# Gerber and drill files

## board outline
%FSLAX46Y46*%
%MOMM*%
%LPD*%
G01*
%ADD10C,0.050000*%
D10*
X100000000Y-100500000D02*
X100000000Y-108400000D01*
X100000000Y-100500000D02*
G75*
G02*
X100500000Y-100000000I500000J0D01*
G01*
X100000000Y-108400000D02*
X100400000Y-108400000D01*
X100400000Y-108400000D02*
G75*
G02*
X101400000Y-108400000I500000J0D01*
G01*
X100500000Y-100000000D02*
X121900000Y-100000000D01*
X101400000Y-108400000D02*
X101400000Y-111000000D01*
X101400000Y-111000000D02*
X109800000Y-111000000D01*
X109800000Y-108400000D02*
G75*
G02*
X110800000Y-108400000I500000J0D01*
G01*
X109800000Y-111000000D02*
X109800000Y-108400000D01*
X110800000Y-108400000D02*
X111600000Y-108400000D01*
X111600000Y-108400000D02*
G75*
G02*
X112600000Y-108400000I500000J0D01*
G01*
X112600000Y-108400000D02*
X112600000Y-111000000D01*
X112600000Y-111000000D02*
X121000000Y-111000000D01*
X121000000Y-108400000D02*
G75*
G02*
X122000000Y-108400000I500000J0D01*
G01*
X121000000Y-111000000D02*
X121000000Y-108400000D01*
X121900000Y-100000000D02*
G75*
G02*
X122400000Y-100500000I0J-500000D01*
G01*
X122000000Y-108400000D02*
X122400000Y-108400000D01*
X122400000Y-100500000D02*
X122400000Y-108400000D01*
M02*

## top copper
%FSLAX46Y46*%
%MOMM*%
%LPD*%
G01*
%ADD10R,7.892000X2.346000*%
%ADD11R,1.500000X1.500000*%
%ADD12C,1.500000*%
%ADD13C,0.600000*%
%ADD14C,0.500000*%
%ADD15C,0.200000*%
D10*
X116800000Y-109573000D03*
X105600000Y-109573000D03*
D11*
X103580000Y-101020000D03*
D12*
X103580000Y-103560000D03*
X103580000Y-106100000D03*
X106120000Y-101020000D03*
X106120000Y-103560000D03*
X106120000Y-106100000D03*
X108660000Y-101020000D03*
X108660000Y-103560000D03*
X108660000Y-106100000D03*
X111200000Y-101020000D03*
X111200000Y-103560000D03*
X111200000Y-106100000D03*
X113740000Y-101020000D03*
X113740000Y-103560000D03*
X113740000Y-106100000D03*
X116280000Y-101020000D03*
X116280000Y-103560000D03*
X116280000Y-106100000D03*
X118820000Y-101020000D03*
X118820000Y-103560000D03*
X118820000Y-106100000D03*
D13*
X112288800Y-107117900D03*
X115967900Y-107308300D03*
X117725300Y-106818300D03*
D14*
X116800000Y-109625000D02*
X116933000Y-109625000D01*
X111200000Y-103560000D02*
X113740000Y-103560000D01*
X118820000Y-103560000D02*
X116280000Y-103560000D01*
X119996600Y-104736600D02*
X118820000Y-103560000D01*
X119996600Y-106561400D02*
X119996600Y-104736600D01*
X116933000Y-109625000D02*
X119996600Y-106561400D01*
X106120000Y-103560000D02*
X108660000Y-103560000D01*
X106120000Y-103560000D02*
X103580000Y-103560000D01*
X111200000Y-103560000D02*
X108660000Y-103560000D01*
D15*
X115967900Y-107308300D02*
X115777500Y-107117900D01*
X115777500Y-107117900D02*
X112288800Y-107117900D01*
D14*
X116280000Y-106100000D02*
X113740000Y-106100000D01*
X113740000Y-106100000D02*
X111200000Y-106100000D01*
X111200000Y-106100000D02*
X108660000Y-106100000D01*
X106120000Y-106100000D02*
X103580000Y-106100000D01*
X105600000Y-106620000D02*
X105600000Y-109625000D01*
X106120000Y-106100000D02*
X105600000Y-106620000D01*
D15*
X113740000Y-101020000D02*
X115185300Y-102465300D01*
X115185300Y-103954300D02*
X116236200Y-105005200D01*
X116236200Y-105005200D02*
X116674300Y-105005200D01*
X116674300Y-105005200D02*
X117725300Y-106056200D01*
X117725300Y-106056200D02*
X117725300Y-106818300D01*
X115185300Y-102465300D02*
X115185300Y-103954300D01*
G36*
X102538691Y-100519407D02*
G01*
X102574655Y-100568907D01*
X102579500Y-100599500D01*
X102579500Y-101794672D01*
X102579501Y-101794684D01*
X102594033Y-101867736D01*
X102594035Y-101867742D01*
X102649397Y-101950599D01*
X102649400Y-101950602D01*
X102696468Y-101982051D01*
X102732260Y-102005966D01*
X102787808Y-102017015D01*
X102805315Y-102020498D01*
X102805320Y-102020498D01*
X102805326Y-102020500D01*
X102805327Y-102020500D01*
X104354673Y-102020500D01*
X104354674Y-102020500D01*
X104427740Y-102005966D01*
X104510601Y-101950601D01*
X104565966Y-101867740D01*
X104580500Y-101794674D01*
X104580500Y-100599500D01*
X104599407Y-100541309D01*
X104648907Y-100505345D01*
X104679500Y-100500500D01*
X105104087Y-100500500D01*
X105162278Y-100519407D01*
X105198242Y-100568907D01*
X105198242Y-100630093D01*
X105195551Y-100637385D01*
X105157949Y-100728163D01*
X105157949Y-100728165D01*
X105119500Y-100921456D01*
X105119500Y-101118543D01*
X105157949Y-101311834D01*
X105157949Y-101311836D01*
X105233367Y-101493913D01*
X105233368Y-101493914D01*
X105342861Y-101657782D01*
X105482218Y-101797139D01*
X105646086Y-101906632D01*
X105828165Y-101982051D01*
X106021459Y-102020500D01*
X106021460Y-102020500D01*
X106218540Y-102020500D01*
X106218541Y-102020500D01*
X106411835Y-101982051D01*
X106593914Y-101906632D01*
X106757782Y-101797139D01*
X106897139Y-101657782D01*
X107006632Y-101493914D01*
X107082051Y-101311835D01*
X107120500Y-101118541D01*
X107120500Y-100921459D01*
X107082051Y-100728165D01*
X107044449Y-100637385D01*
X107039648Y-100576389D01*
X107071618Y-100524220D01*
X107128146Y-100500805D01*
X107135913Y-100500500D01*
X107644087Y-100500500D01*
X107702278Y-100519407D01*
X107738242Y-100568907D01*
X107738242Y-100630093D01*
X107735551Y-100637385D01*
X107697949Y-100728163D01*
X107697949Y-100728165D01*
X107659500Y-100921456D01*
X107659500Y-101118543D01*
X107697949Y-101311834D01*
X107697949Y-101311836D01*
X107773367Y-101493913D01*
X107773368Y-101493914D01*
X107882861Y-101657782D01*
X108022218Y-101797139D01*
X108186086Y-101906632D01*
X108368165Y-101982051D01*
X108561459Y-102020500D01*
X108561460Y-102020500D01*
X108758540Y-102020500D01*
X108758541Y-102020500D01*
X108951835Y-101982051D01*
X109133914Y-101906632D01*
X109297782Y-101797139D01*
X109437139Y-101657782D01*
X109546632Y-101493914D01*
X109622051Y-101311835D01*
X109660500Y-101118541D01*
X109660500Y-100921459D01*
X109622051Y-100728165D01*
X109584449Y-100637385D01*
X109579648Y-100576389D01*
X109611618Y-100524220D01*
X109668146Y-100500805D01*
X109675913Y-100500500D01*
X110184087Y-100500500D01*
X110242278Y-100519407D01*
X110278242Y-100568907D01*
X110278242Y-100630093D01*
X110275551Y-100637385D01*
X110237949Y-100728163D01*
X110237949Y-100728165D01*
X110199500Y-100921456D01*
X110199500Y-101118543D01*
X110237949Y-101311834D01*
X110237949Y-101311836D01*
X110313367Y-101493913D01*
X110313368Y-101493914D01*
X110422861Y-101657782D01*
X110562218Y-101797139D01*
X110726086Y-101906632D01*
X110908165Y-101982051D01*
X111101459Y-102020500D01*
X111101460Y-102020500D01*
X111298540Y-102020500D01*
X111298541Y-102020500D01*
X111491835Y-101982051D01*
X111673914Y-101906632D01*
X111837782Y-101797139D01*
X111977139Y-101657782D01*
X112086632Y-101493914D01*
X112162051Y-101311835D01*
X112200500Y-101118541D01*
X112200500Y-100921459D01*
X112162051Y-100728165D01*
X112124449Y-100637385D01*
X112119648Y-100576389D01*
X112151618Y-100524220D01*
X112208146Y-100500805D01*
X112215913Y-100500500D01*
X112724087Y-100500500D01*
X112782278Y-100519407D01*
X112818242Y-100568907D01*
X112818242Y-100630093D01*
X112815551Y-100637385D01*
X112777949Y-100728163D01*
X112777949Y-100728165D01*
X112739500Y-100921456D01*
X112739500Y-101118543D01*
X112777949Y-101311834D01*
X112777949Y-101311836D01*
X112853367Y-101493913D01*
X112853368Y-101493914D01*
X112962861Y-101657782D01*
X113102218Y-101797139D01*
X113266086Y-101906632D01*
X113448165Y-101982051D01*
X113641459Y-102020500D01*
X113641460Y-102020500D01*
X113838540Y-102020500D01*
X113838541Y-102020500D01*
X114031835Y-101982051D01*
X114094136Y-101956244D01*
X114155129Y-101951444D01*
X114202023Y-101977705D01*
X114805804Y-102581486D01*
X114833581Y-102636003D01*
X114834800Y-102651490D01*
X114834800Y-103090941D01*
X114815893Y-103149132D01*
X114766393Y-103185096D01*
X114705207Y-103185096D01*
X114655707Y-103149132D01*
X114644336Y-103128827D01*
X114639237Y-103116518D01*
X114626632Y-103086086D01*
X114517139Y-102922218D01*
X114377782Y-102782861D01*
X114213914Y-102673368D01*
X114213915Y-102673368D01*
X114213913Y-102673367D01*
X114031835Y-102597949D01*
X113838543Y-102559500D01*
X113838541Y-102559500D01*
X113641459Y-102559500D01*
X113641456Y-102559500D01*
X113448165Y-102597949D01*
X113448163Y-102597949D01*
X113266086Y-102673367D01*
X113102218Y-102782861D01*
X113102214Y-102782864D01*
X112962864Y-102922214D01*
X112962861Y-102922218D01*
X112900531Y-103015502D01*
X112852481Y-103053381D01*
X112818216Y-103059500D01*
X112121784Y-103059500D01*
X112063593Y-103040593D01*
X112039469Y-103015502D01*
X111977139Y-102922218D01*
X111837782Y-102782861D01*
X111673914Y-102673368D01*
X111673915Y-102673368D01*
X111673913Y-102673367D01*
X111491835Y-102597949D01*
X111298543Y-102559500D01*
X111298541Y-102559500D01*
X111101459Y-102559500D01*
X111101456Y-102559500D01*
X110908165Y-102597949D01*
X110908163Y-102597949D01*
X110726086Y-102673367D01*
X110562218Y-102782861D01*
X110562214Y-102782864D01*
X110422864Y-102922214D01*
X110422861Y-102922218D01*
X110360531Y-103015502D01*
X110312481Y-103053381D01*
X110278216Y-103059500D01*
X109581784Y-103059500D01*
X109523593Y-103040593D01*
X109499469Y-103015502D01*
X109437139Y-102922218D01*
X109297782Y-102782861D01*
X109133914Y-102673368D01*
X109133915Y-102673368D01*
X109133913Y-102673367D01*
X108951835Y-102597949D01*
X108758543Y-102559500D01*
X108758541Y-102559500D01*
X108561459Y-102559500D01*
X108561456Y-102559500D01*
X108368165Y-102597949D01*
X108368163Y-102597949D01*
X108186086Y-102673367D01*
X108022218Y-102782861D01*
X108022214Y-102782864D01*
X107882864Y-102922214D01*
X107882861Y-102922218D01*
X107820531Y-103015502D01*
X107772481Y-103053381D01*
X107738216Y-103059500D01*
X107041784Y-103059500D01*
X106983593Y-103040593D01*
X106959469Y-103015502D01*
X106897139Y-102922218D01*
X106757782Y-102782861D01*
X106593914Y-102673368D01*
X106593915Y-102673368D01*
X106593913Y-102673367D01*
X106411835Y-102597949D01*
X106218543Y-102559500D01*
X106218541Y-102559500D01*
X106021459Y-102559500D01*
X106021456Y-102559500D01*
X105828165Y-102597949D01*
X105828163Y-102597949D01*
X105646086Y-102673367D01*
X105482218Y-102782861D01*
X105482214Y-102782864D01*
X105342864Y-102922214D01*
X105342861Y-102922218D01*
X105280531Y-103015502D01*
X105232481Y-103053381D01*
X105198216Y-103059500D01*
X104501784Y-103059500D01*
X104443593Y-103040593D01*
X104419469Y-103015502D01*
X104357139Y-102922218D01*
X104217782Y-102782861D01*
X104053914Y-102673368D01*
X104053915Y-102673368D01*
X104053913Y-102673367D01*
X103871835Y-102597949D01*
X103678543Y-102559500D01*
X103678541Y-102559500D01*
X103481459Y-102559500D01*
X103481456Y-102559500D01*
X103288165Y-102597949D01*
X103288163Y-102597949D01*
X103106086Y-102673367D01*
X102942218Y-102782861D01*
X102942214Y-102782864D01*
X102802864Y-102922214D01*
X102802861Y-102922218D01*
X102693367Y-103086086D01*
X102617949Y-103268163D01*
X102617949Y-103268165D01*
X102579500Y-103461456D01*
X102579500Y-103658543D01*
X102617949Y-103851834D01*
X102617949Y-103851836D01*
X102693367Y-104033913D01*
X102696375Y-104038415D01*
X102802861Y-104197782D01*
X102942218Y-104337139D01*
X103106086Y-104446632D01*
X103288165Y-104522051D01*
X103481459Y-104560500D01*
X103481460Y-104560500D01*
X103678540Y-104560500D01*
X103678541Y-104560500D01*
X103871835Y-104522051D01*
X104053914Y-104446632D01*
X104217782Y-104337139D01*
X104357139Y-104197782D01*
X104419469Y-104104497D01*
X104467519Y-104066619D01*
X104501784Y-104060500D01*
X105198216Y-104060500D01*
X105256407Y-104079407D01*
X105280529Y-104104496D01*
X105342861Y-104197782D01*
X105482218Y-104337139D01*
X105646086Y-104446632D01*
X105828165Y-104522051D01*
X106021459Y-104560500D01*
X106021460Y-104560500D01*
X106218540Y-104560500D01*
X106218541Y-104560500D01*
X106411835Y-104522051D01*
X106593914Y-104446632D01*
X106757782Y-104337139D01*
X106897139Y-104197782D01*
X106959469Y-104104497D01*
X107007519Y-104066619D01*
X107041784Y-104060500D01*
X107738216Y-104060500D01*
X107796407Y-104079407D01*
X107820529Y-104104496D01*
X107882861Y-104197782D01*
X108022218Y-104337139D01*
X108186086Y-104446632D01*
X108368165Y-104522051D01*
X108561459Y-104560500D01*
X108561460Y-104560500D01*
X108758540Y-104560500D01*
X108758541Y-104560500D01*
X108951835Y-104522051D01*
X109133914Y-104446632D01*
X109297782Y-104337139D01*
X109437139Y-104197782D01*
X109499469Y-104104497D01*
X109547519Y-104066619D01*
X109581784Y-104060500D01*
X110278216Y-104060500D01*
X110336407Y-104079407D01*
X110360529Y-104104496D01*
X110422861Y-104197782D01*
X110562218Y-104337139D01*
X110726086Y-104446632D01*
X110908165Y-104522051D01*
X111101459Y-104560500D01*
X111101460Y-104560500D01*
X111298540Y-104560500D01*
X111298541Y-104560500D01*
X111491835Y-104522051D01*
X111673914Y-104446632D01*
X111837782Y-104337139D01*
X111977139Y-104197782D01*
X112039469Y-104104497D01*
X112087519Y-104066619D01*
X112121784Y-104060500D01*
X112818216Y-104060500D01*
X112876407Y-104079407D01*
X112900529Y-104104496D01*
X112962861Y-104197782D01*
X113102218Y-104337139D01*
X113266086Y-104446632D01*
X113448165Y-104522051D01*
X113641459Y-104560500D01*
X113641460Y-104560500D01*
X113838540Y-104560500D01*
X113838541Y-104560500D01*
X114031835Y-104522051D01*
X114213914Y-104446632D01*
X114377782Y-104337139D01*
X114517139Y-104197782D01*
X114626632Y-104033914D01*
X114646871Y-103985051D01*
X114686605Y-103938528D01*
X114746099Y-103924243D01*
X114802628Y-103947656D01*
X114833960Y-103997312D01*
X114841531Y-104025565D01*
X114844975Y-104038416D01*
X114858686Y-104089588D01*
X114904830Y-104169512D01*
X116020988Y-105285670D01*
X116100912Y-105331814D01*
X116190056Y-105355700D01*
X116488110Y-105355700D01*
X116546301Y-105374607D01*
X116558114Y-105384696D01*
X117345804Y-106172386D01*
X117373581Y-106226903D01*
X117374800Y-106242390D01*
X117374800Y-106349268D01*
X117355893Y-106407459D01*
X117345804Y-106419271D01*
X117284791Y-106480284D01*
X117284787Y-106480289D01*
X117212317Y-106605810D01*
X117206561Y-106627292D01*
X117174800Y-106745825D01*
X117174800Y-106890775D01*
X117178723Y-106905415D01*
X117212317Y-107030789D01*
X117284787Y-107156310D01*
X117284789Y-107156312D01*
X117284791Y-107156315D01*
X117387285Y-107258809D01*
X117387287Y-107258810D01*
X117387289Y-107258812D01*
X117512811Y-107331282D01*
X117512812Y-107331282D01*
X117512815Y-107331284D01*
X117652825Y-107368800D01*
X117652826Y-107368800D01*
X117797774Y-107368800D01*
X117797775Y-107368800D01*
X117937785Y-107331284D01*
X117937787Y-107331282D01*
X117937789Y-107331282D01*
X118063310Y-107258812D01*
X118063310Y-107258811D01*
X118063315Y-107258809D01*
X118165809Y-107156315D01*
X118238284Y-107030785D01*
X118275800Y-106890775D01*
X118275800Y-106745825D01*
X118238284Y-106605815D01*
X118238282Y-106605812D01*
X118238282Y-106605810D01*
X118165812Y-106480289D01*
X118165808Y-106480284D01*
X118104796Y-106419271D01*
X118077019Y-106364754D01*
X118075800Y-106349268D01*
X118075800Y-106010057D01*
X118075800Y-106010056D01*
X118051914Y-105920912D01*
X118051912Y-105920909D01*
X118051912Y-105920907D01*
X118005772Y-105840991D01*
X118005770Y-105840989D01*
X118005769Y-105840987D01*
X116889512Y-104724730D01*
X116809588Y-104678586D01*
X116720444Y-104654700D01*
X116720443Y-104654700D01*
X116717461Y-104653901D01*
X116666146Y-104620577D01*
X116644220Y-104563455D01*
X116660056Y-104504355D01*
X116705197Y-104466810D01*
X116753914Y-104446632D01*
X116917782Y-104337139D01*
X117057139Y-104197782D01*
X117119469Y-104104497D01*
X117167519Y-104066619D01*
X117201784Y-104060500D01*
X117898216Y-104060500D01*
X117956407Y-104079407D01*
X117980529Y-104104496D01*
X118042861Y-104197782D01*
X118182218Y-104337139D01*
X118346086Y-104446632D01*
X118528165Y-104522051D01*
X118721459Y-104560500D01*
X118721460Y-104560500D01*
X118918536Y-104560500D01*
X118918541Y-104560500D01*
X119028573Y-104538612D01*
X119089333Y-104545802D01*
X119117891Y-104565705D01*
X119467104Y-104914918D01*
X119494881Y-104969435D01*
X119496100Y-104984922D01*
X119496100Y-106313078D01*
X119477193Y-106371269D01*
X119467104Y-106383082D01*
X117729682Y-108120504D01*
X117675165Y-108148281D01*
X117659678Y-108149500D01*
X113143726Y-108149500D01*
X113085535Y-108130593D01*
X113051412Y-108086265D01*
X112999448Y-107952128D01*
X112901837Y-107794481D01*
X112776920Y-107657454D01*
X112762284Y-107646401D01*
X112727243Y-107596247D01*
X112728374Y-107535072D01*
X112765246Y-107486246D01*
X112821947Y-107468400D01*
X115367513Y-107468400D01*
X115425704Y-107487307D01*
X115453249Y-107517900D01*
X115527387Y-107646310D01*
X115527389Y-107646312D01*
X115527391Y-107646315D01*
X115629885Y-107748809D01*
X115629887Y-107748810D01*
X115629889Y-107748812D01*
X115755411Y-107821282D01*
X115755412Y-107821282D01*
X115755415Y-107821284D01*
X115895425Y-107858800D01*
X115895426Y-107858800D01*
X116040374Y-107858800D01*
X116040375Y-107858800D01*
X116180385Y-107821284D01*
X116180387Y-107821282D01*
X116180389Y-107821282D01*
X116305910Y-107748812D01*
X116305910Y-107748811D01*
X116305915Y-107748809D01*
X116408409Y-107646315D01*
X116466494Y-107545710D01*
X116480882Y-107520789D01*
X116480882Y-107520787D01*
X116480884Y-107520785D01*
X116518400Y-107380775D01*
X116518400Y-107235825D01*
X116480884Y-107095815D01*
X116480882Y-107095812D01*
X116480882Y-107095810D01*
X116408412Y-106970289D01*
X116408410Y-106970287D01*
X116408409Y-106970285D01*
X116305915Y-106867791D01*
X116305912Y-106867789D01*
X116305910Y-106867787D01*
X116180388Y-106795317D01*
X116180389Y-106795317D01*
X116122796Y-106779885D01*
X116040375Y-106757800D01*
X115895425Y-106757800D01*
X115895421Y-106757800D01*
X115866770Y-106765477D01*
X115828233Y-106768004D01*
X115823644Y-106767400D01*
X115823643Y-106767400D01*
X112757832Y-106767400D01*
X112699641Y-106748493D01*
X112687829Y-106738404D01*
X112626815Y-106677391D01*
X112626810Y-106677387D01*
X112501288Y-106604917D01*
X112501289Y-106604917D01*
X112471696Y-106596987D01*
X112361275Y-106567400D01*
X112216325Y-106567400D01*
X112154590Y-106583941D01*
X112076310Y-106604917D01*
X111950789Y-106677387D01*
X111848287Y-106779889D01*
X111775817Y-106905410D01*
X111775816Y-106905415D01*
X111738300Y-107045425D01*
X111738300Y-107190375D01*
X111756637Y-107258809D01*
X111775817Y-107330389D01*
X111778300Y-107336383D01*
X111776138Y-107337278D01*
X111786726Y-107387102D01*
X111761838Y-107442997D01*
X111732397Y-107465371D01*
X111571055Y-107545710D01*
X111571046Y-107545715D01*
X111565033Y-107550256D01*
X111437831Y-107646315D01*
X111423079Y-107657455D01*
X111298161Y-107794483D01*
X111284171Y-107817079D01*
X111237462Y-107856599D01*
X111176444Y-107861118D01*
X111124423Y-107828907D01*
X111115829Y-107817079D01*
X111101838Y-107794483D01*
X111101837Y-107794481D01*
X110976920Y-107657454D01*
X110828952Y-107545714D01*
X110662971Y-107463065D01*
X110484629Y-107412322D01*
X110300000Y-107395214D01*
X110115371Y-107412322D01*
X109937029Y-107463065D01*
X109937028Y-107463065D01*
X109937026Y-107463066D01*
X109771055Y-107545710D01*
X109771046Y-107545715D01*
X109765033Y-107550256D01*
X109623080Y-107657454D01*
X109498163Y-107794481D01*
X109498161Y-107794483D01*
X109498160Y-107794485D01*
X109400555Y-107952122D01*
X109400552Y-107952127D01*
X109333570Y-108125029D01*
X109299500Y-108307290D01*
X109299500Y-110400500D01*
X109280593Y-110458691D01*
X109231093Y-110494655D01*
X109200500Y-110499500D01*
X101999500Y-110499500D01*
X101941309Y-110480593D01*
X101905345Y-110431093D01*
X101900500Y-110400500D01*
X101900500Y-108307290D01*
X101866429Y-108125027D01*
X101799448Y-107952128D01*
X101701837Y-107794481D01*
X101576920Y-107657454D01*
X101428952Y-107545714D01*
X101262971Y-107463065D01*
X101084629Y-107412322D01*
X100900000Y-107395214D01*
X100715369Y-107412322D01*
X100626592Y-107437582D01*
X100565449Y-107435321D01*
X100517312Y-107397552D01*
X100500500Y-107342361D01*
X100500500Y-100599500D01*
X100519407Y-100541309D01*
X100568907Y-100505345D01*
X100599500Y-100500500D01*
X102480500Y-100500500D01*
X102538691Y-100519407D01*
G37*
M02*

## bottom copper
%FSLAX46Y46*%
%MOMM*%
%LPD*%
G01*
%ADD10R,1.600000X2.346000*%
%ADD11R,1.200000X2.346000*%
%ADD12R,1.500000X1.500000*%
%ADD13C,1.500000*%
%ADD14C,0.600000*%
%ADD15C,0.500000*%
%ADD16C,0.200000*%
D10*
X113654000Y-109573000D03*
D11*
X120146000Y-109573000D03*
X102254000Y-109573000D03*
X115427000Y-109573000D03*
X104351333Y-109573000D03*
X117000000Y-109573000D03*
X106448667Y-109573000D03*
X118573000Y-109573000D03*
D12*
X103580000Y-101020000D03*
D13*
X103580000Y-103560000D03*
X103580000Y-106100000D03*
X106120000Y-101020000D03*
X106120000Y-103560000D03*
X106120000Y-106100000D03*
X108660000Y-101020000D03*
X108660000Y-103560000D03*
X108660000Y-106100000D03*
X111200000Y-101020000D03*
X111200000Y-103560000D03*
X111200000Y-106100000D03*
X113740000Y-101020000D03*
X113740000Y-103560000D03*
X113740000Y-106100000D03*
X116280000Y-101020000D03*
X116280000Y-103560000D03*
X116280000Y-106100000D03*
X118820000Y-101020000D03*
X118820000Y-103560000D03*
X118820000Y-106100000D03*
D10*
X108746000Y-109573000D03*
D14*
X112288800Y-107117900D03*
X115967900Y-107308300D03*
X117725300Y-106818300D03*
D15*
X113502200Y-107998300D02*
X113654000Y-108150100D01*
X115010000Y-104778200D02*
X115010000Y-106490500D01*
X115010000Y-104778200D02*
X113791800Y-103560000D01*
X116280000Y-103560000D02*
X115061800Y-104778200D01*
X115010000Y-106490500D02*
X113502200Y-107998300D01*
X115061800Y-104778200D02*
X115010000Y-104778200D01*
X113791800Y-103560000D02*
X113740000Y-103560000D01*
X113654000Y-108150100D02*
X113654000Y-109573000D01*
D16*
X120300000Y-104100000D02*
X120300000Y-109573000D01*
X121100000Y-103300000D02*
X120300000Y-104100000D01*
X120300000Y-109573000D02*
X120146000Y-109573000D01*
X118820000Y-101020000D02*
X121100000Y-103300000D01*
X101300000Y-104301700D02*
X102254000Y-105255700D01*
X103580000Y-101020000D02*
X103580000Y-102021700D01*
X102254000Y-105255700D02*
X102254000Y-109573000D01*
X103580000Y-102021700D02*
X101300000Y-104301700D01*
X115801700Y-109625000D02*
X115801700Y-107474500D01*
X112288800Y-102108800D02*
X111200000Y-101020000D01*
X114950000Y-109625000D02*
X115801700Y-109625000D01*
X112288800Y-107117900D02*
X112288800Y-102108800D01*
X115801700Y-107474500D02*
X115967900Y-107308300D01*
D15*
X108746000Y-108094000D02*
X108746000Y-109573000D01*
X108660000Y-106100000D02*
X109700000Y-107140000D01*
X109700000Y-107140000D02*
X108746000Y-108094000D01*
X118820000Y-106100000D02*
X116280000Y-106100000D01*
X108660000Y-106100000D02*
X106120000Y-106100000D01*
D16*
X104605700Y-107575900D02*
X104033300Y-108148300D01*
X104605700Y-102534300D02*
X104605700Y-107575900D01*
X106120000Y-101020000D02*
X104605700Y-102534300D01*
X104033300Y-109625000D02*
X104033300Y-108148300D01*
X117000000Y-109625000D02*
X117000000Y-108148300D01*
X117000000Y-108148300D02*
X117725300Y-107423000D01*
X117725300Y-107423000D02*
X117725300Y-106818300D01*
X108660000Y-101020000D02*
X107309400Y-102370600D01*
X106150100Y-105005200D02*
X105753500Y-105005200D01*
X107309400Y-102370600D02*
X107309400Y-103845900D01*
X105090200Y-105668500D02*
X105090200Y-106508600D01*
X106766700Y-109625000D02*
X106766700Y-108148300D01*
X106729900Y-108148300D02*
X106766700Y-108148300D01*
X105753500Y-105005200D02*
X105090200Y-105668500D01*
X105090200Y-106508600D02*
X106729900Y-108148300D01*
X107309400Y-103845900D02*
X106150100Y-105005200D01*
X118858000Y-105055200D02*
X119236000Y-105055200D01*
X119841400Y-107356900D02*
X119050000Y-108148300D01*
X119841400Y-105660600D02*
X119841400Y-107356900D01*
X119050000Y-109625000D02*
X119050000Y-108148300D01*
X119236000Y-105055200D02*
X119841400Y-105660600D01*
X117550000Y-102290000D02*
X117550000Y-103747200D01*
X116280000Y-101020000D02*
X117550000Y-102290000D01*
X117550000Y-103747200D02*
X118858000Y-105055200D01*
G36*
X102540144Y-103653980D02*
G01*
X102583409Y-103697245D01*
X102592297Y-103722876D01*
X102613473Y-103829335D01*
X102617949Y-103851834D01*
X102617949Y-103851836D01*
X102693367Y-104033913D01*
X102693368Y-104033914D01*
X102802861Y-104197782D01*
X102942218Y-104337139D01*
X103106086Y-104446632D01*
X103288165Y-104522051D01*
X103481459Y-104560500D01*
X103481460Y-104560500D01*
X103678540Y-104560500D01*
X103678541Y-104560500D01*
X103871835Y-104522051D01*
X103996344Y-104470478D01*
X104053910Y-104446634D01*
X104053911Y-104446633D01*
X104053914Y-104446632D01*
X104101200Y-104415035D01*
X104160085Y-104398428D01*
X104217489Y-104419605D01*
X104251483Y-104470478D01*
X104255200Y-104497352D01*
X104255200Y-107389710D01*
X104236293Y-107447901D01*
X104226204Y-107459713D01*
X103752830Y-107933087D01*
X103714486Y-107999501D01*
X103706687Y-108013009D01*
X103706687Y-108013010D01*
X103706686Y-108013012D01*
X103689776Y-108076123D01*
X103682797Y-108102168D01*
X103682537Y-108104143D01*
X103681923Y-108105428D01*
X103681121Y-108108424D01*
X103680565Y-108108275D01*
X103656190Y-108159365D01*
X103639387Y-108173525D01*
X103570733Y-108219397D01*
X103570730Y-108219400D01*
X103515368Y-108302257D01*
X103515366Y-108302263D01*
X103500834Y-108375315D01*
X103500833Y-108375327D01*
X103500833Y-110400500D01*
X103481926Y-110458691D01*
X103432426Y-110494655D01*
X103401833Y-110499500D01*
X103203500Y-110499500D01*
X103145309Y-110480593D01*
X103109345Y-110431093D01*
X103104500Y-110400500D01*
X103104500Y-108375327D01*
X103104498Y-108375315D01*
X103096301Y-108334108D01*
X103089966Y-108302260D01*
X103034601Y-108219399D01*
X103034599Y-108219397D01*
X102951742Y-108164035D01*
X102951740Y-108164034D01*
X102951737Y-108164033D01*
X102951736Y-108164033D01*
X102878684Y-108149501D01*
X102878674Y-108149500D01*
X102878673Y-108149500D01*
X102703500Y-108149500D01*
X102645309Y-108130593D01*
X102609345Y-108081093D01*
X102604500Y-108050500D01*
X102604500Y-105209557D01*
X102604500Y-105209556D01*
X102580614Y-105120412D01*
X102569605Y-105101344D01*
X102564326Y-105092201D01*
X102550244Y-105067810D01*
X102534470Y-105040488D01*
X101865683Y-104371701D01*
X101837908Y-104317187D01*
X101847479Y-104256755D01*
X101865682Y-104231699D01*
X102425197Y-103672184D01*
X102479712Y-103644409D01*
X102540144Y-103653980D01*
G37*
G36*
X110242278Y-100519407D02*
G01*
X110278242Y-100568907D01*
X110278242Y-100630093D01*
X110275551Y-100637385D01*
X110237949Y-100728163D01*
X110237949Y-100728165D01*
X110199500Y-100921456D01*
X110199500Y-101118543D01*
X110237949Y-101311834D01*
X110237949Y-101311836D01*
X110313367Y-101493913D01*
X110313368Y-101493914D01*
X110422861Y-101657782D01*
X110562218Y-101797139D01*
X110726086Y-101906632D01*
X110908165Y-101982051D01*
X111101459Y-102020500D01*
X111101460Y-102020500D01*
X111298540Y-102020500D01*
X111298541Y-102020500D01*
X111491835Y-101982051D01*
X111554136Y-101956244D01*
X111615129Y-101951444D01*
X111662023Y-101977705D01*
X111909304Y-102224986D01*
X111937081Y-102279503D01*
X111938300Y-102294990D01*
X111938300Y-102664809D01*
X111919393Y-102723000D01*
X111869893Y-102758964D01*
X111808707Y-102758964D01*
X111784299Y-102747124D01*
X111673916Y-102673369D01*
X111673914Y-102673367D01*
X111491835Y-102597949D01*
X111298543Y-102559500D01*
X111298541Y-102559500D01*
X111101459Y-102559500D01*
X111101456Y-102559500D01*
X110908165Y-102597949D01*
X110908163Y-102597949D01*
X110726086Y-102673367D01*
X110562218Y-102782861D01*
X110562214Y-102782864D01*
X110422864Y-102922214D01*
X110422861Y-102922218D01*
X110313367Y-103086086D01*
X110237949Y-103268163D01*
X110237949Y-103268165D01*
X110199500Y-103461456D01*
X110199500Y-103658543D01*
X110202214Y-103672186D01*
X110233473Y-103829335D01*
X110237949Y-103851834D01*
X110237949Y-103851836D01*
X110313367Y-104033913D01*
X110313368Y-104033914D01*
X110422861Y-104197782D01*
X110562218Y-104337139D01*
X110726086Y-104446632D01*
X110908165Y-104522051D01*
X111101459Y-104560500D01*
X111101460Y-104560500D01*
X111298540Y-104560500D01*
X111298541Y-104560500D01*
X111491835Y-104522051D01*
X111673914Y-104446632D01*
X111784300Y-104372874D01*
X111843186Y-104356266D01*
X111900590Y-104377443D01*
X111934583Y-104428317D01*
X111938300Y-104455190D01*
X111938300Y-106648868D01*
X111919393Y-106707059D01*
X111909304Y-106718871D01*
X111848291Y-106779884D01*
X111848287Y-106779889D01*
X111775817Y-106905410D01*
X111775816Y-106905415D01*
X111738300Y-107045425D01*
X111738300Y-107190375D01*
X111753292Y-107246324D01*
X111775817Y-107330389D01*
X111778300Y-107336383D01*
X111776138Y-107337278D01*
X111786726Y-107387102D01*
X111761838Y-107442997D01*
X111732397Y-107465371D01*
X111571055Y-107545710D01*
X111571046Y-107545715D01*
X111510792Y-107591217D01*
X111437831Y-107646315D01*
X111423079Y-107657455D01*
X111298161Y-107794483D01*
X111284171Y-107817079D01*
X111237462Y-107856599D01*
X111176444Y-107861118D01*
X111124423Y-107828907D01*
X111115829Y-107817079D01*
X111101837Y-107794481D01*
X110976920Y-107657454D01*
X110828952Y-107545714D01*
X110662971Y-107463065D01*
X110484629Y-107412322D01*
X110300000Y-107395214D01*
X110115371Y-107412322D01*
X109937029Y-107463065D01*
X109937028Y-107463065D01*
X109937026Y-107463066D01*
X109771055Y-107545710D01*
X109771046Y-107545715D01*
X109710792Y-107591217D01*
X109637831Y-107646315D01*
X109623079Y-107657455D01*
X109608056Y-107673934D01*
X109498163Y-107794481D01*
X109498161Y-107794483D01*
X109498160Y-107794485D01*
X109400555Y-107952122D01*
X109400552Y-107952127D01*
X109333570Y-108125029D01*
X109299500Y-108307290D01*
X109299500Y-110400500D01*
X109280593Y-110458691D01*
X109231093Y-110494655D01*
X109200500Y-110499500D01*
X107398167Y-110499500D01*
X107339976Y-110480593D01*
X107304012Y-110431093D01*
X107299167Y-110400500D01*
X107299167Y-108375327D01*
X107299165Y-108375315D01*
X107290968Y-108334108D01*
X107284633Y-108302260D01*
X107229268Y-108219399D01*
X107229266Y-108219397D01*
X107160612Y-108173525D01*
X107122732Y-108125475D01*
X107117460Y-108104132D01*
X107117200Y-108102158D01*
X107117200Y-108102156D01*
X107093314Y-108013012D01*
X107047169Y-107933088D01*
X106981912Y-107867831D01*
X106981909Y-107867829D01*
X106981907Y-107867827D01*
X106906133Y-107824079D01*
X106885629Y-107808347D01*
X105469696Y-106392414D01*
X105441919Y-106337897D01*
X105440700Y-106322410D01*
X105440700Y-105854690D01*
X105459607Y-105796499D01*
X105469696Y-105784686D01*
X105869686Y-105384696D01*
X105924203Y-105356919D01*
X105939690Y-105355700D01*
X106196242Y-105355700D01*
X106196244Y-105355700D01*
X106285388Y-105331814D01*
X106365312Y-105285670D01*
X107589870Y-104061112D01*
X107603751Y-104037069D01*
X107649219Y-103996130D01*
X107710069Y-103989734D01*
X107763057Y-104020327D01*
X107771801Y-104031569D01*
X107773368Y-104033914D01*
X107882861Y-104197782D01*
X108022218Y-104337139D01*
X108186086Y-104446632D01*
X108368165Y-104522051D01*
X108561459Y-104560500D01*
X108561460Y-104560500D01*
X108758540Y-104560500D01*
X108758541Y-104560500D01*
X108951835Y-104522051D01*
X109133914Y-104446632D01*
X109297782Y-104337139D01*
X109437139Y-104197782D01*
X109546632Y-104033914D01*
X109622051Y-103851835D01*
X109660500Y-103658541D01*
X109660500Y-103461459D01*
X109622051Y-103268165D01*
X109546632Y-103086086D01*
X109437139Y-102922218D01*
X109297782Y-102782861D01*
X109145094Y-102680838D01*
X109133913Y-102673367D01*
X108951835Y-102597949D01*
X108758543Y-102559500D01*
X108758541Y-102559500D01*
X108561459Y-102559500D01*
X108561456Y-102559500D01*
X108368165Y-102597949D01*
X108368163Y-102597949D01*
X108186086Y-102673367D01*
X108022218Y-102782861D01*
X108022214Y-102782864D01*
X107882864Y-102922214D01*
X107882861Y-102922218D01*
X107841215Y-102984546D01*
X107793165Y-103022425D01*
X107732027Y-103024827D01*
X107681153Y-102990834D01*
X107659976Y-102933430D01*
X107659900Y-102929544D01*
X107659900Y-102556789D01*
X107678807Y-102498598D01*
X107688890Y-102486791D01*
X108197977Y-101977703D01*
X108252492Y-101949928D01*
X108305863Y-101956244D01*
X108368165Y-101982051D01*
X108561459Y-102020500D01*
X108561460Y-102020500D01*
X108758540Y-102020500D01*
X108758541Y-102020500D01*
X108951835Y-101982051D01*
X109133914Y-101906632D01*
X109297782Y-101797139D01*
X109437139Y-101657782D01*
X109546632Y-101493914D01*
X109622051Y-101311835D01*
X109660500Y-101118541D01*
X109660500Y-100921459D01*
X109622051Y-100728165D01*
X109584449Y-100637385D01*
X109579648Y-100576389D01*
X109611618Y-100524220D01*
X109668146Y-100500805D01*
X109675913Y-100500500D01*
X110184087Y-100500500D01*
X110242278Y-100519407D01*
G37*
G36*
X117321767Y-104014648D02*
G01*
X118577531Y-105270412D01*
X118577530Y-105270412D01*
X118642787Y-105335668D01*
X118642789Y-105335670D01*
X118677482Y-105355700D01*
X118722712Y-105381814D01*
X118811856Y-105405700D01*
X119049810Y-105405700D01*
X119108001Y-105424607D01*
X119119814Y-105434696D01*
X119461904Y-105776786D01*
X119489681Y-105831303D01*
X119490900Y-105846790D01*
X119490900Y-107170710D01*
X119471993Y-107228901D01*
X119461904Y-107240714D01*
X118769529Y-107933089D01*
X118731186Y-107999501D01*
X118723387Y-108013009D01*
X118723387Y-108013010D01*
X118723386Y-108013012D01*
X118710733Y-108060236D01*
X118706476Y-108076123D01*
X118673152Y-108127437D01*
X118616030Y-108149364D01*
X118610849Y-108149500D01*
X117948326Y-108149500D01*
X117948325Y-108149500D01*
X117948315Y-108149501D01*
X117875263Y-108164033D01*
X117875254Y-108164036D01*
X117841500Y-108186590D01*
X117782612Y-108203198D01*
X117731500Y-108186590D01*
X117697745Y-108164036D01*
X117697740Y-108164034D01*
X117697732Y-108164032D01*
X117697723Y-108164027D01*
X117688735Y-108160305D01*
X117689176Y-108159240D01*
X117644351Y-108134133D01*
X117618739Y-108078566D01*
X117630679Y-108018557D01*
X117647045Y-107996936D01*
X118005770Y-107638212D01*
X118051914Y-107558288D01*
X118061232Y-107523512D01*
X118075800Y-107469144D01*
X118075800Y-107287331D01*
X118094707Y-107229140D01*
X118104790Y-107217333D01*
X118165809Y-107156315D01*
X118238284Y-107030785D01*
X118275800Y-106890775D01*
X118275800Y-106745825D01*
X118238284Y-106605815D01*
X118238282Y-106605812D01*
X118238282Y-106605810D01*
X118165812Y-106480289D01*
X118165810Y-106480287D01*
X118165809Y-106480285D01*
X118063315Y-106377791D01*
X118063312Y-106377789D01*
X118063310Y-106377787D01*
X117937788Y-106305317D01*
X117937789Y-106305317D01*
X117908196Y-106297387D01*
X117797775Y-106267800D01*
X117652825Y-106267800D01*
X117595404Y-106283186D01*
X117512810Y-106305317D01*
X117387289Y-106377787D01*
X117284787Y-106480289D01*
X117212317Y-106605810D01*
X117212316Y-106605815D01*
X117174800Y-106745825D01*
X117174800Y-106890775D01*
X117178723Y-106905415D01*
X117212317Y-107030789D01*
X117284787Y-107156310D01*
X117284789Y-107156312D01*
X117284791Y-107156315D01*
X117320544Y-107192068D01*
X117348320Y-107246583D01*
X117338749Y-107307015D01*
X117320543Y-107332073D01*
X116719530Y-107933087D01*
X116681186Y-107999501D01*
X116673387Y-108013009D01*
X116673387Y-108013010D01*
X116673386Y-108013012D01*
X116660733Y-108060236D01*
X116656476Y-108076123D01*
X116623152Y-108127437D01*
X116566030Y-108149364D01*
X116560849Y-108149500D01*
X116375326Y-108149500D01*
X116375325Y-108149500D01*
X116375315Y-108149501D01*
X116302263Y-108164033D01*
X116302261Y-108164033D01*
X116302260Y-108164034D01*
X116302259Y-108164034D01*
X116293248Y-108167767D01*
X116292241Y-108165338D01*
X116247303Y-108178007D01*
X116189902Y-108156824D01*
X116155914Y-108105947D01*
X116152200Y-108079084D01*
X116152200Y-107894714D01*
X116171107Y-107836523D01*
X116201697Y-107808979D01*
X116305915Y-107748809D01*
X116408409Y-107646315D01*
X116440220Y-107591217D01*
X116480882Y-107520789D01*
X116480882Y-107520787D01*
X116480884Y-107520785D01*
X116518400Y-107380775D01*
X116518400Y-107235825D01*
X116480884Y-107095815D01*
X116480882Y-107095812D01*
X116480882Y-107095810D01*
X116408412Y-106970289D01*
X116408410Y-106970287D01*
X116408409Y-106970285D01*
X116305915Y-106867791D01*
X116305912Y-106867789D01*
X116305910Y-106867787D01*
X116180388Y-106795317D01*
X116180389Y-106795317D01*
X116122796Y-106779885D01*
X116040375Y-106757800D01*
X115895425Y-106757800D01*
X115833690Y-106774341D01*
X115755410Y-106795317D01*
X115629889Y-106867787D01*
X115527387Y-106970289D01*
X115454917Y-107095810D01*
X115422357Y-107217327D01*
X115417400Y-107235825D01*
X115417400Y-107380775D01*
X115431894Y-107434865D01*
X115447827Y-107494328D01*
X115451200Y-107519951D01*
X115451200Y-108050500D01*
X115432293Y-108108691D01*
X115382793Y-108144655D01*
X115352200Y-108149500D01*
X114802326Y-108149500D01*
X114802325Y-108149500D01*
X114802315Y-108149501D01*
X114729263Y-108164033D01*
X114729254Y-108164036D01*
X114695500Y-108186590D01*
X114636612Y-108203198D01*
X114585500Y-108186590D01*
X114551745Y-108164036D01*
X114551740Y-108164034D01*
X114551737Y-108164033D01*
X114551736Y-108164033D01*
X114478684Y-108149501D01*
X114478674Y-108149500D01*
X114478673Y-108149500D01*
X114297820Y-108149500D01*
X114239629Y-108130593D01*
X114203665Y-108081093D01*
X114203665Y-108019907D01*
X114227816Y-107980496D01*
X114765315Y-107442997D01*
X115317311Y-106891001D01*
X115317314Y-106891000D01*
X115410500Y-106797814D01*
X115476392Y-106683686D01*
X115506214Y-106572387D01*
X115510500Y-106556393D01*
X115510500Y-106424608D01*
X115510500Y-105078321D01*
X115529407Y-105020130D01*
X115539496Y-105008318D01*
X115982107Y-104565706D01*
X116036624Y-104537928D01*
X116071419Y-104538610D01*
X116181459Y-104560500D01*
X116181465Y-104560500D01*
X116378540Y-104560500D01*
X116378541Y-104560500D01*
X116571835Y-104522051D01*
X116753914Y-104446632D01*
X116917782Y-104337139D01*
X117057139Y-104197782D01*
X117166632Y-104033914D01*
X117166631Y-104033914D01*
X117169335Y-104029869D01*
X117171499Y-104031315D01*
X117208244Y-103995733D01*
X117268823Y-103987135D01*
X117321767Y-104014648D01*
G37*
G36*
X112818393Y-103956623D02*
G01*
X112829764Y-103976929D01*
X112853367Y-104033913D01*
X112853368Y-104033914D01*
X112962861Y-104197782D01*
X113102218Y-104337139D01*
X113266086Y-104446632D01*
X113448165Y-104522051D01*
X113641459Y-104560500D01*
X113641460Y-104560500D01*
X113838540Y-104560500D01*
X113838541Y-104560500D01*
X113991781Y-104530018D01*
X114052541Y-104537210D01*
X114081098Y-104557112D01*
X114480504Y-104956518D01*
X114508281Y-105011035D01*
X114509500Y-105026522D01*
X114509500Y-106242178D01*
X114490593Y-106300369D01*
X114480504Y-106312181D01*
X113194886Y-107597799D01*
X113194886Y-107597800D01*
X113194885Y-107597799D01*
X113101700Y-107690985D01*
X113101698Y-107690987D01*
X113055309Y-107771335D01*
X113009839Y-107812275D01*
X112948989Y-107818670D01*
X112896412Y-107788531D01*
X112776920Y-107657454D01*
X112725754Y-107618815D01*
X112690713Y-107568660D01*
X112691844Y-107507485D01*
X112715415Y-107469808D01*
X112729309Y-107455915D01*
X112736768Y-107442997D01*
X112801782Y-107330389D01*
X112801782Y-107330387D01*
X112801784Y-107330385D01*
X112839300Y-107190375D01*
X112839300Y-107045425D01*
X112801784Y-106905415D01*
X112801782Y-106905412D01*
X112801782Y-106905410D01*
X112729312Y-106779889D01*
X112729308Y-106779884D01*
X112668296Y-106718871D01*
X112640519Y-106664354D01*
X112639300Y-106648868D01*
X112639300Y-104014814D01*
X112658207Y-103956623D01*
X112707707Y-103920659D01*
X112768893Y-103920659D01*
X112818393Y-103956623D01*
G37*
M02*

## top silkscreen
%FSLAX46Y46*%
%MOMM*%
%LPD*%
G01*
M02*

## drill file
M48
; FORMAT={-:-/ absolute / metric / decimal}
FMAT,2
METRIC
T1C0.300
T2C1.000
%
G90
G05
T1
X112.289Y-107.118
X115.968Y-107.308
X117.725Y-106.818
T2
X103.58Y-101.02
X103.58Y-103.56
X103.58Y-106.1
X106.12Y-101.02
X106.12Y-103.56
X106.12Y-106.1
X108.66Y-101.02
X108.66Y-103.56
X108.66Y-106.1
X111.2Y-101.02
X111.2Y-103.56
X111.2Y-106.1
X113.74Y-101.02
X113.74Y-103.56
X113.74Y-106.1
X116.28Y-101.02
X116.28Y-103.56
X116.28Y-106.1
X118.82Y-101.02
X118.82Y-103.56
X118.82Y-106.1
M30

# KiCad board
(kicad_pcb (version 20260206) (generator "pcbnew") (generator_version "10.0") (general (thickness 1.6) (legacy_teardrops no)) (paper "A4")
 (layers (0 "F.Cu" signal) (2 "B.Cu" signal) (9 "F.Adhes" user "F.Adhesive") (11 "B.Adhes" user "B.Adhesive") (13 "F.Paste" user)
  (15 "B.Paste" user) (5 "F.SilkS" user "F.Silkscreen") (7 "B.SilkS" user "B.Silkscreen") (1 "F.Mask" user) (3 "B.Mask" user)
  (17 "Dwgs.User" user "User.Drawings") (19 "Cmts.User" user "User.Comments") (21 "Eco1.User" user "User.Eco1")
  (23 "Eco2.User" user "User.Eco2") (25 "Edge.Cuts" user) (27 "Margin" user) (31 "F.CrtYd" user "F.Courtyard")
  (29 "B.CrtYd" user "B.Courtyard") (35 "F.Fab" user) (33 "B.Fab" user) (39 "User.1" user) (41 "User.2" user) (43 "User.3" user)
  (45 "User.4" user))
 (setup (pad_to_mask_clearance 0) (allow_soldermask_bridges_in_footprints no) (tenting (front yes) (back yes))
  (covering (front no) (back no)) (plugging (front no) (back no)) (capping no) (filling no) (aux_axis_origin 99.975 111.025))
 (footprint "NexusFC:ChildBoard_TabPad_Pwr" (layer "F.Cu") (at 113.654 108.4)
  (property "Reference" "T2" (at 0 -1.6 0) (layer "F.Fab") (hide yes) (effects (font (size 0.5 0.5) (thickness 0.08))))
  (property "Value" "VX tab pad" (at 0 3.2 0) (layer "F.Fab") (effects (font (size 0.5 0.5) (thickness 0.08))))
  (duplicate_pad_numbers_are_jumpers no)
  (pad "1" smd rect (at 0 1.173) (size 1.6 2.346) (layers "B.Cu" "B.Mask") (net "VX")))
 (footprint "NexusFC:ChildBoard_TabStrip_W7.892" (layer "F.Cu") (at 116.8 108.4)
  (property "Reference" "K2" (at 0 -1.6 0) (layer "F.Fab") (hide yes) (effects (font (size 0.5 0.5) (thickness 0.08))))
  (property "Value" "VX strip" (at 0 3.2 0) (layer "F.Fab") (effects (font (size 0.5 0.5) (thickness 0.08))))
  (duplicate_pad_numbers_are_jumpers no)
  (pad "1" smd rect (at 0 1.173) (size 7.892 2.346) (layers "F.Cu" "F.Mask") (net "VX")))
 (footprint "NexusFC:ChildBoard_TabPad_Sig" (layer "F.Cu") (at 120.146 108.4)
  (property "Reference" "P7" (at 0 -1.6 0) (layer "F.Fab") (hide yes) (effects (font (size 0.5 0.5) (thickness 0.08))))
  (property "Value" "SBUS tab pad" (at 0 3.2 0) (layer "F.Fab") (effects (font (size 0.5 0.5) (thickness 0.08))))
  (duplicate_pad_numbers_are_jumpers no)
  (pad "1" smd rect (at 0 1.173) (size 1.2 2.346) (layers "B.Cu" "B.Mask") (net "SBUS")))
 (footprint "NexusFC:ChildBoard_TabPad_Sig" (layer "F.Cu") (at 102.254 108.4)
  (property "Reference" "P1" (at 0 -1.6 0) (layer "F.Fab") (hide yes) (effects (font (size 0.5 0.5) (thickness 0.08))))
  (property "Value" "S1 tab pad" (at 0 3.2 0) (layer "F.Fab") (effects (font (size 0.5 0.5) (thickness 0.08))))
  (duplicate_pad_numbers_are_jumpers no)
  (pad "1" smd rect (at 0 1.173) (size 1.2 2.346) (layers "B.Cu" "B.Mask") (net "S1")))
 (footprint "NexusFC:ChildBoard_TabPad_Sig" (layer "F.Cu") (at 115.427 108.4)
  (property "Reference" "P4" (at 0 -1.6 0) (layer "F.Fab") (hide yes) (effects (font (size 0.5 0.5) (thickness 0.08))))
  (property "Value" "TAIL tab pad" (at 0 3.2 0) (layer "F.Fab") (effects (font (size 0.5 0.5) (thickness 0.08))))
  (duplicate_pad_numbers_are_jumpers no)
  (pad "1" smd rect (at 0 1.173) (size 1.2 2.346) (layers "B.Cu" "B.Mask") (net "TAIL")))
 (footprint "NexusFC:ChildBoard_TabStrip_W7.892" (layer "F.Cu") (at 105.6 108.4)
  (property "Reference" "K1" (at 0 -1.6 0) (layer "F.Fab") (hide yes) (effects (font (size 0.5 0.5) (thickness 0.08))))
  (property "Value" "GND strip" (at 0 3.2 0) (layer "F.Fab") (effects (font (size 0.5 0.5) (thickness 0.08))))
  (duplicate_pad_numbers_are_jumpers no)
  (pad "1" smd rect (at 0 1.173) (size 7.892 2.346) (layers "F.Cu" "F.Mask") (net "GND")))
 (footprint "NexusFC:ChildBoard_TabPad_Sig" (layer "F.Cu") (at 104.351333 108.4)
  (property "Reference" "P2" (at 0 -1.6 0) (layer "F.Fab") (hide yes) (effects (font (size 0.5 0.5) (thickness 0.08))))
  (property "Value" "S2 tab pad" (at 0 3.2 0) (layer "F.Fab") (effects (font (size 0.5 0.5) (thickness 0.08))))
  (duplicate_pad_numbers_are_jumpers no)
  (pad "1" smd rect (at 0 1.173) (size 1.2 2.346) (layers "B.Cu" "B.Mask") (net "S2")))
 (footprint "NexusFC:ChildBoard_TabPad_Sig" (layer "F.Cu") (at 117 108.4)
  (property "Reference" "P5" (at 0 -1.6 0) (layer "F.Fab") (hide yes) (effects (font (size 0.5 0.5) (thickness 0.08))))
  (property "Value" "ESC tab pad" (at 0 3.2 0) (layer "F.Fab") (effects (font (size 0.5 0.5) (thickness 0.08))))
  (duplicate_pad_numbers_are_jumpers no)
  (pad "1" smd rect (at 0 1.173) (size 1.2 2.346) (layers "B.Cu" "B.Mask") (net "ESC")))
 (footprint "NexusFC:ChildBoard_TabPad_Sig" (layer "F.Cu") (at 106.448667 108.4)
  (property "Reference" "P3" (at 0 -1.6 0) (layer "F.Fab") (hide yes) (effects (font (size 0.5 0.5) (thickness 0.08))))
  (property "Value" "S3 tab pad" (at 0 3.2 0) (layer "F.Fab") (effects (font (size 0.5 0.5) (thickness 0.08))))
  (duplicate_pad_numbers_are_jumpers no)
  (pad "1" smd rect (at 0 1.173) (size 1.2 2.346) (layers "B.Cu" "B.Mask") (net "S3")))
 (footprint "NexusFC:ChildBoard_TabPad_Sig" (layer "F.Cu") (at 118.573 108.4)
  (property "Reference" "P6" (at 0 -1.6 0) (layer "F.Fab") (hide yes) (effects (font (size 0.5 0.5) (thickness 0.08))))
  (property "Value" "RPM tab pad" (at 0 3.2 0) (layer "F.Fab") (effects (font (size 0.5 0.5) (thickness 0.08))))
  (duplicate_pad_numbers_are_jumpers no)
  (pad "1" smd rect (at 0 1.173) (size 1.2 2.346) (layers "B.Cu" "B.Mask") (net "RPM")))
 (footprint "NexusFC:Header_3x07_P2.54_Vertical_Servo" (layer "F.Cu") (at 111.2 103.56)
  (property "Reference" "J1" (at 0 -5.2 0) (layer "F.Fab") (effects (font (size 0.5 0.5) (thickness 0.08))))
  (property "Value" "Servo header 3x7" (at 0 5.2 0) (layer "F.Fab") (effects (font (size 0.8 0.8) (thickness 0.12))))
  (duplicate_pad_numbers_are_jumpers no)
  (pad "1" thru_hole rect (at -7.62 -2.54) (size 1.5 1.5) (drill 1) (layers "*.Cu" "*.Mask") (remove_unused_layers no) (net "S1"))
  (pad "2" thru_hole circle (at -7.62 0) (size 1.5 1.5) (drill 1) (layers "*.Cu" "*.Mask") (remove_unused_layers no) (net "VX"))
  (pad "3" thru_hole circle (at -7.62 2.54) (size 1.5 1.5) (drill 1) (layers "*.Cu" "*.Mask") (remove_unused_layers no) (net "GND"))
  (pad "4" thru_hole circle (at -5.08 -2.54) (size 1.5 1.5) (drill 1) (layers "*.Cu" "*.Mask") (remove_unused_layers no) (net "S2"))
  (pad "5" thru_hole circle (at -5.08 0) (size 1.5 1.5) (drill 1) (layers "*.Cu" "*.Mask") (remove_unused_layers no) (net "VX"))
  (pad "6" thru_hole circle (at -5.08 2.54) (size 1.5 1.5) (drill 1) (layers "*.Cu" "*.Mask") (remove_unused_layers no) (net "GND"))
  (pad "7" thru_hole circle (at -2.54 -2.54) (size 1.5 1.5) (drill 1) (layers "*.Cu" "*.Mask") (remove_unused_layers no) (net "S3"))
  (pad "8" thru_hole circle (at -2.54 0) (size 1.5 1.5) (drill 1) (layers "*.Cu" "*.Mask") (remove_unused_layers no) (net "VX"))
  (pad "9" thru_hole circle (at -2.54 2.54) (size 1.5 1.5) (drill 1) (layers "*.Cu" "*.Mask") (remove_unused_layers no) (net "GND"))
  (pad "10" thru_hole circle (at 0 -2.54) (size 1.5 1.5) (drill 1) (layers "*.Cu" "*.Mask") (remove_unused_layers no) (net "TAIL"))
  (pad "11" thru_hole circle (at 0 0) (size 1.5 1.5) (drill 1) (layers "*.Cu" "*.Mask") (remove_unused_layers no) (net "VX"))
  (pad "12" thru_hole circle (at 0 2.54) (size 1.5 1.5) (drill 1) (layers "*.Cu" "*.Mask") (remove_unused_layers no) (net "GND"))
  (pad "13" thru_hole circle (at 2.54 -2.54) (size 1.5 1.5) (drill 1) (layers "*.Cu" "*.Mask") (remove_unused_layers no) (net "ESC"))
  (pad "14" thru_hole circle (at 2.54 0) (size 1.5 1.5) (drill 1) (layers "*.Cu" "*.Mask") (remove_unused_layers no) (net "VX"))
  (pad "15" thru_hole circle (at 2.54 2.54) (size 1.5 1.5) (drill 1) (layers "*.Cu" "*.Mask") (remove_unused_layers no) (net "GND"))
  (pad "16" thru_hole circle (at 5.08 -2.54) (size 1.5 1.5) (drill 1) (layers "*.Cu" "*.Mask") (remove_unused_layers no) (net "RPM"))
  (pad "17" thru_hole circle (at 5.08 0) (size 1.5 1.5) (drill 1) (layers "*.Cu" "*.Mask") (remove_unused_layers no) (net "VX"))
  (pad "18" thru_hole circle (at 5.08 2.54) (size 1.5 1.5) (drill 1) (layers "*.Cu" "*.Mask") (remove_unused_layers no) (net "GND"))
  (pad "19" thru_hole circle (at 7.62 -2.54) (size 1.5 1.5) (drill 1) (layers "*.Cu" "*.Mask") (remove_unused_layers no) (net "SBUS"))
  (pad "20" thru_hole circle (at 7.62 0) (size 1.5 1.5) (drill 1) (layers "*.Cu" "*.Mask") (remove_unused_layers no) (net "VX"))
  (pad "21" thru_hole circle (at 7.62 2.54) (size 1.5 1.5) (drill 1) (layers "*.Cu" "*.Mask") (remove_unused_layers no) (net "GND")))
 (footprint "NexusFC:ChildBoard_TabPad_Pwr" (layer "F.Cu") (at 108.746 108.4)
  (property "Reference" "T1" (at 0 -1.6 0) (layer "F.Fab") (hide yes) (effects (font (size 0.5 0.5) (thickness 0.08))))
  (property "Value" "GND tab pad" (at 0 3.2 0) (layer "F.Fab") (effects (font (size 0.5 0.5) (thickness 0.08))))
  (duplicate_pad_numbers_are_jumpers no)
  (pad "1" smd rect (at 0 1.173) (size 1.6 2.346) (layers "B.Cu" "B.Mask") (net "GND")))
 (gr_line (start 100 100.5) (end 100 108.4) (stroke (width 0.05) (type default)) (layer "Edge.Cuts"))
 (gr_arc (start 100 100.5) (mid 100.146447 100.146447) (end 100.5 100) (stroke (width 0.05) (type default)) (layer "Edge.Cuts"))
 (gr_line (start 100 108.4) (end 100.4 108.4) (stroke (width 0.05) (type solid)) (layer "Edge.Cuts"))
 (gr_arc (start 100.4 108.4) (mid 100.9 107.9) (end 101.4 108.4) (stroke (width 0.05) (type solid)) (layer "Edge.Cuts"))
 (gr_line (start 100.5 100) (end 121.9 100) (stroke (width 0.05) (type default)) (layer "Edge.Cuts"))
 (gr_line (start 101.4 108.4) (end 101.4 111) (stroke (width 0.05) (type solid)) (layer "Edge.Cuts"))
 (gr_line (start 101.4 111) (end 109.8 111) (stroke (width 0.05) (type solid)) (layer "Edge.Cuts"))
 (gr_arc (start 109.8 108.4) (mid 110.3 107.9) (end 110.8 108.4) (stroke (width 0.05) (type solid)) (layer "Edge.Cuts"))
 (gr_line (start 109.8 111) (end 109.8 108.4) (stroke (width 0.05) (type solid)) (layer "Edge.Cuts"))
 (gr_line (start 110.8 108.4) (end 111.6 108.4) (stroke (width 0.05) (type solid)) (layer "Edge.Cuts"))
 (gr_arc (start 111.6 108.4) (mid 112.1 107.9) (end 112.6 108.4) (stroke (width 0.05) (type solid)) (layer "Edge.Cuts"))
 (gr_line (start 112.6 108.4) (end 112.6 111) (stroke (width 0.05) (type solid)) (layer "Edge.Cuts"))
 (gr_line (start 112.6 111) (end 121 111) (stroke (width 0.05) (type solid)) (layer "Edge.Cuts"))
 (gr_arc (start 121 108.4) (mid 121.5 107.9) (end 122 108.4) (stroke (width 0.05) (type solid)) (layer "Edge.Cuts"))
 (gr_line (start 121 111) (end 121 108.4) (stroke (width 0.05) (type solid)) (layer "Edge.Cuts"))
 (gr_arc (start 121.9 100) (mid 122.253553 100.146447) (end 122.4 100.5) (stroke (width 0.05) (type default)) (layer "Edge.Cuts"))
 (gr_line (start 122 108.4) (end 122.4 108.4) (stroke (width 0.05) (type solid)) (layer "Edge.Cuts"))
 (gr_line (start 122.4 100.5) (end 122.4 108.4) (stroke (width 0.05) (type default)) (layer "Edge.Cuts"))
 (segment (start 116.8 109.625) (end 116.933 109.625) (width 0.5) (layer "F.Cu") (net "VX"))
 (segment (start 111.2 103.56) (end 113.74 103.56) (width 0.5) (layer "F.Cu") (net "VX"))
 (segment (start 118.82 103.56) (end 116.28 103.56) (width 0.5) (layer "F.Cu") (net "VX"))
 (segment (start 119.9966 104.7366) (end 118.82 103.56) (width 0.5) (layer "F.Cu") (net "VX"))
 (segment (start 119.9966 106.5614) (end 119.9966 104.7366) (width 0.5) (layer "F.Cu") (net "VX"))
 (segment (start 116.933 109.625) (end 119.9966 106.5614) (width 0.5) (layer "F.Cu") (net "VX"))
 (segment (start 106.12 103.56) (end 108.66 103.56) (width 0.5) (layer "F.Cu") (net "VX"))
 (segment (start 106.12 103.56) (end 103.58 103.56) (width 0.5) (layer "F.Cu") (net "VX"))
 (segment (start 111.2 103.56) (end 108.66 103.56) (width 0.5) (layer "F.Cu") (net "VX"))
 (segment (start 113.5022 107.9983) (end 113.654 108.1501) (width 0.5) (layer "B.Cu") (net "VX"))
 (segment (start 115.01 104.7782) (end 115.01 106.4905) (width 0.5) (layer "B.Cu") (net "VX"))
 (segment (start 115.01 104.7782) (end 113.7918 103.56) (width 0.5) (layer "B.Cu") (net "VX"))
 (segment (start 116.28 103.56) (end 115.0618 104.7782) (width 0.5) (layer "B.Cu") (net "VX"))
 (segment (start 115.01 106.4905) (end 113.5022 107.9983) (width 0.5) (layer "B.Cu") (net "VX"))
 (segment (start 115.0618 104.7782) (end 115.01 104.7782) (width 0.5) (layer "B.Cu") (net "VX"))
 (segment (start 113.7918 103.56) (end 113.74 103.56) (width 0.5) (layer "B.Cu") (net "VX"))
 (segment (start 113.654 108.1501) (end 113.654 109.573) (width 0.5) (layer "B.Cu") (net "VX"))
 (segment (start 120.3 104.1) (end 120.3 109.573) (width 0.2) (layer "B.Cu") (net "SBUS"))
 (segment (start 121.1 103.3) (end 120.3 104.1) (width 0.2) (layer "B.Cu") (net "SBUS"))
 (segment (start 120.3 109.573) (end 120.146 109.573) (width 0.2) (layer "B.Cu") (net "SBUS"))
 (segment (start 118.82 101.02) (end 121.1 103.3) (width 0.2) (layer "B.Cu") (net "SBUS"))
 (segment (start 101.3 104.3017) (end 102.254 105.2557) (width 0.2) (layer "B.Cu") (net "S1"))
 (segment (start 103.58 101.02) (end 103.58 102.0217) (width 0.2) (layer "B.Cu") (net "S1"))
 (segment (start 102.254 105.2557) (end 102.254 109.573) (width 0.2) (layer "B.Cu") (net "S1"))
 (segment (start 103.58 102.0217) (end 101.3 104.3017) (width 0.2) (layer "B.Cu") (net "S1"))
 (segment (start 115.9679 107.3083) (end 115.7775 107.1179) (width 0.2) (layer "F.Cu") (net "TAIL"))
 (segment (start 115.7775 107.1179) (end 112.2888 107.1179) (width 0.2) (layer "F.Cu") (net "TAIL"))
 (via (at 112.2888 107.1179) (size 0.6) (drill 0.3) (layers "F.Cu" "B.Cu") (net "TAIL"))
 (via (at 115.9679 107.3083) (size 0.6) (drill 0.3) (layers "F.Cu" "B.Cu") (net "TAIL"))
 (segment (start 115.8017 109.625) (end 115.8017 107.4745) (width 0.2) (layer "B.Cu") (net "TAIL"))
 (segment (start 112.2888 102.1088) (end 111.2 101.02) (width 0.2) (layer "B.Cu") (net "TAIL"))
 (segment (start 114.95 109.625) (end 115.8017 109.625) (width 0.2) (layer "B.Cu") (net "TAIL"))
 (segment (start 112.2888 107.1179) (end 112.2888 102.1088) (width 0.2) (layer "B.Cu") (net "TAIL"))
 (segment (start 115.8017 107.4745) (end 115.9679 107.3083) (width 0.2) (layer "B.Cu") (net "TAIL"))
 (segment (start 116.28 106.1) (end 113.74 106.1) (width 0.5) (layer "F.Cu") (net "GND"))
 (segment (start 113.74 106.1) (end 111.2 106.1) (width 0.5) (layer "F.Cu") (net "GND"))
 (segment (start 111.2 106.1) (end 108.66 106.1) (width 0.5) (layer "F.Cu") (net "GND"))
 (segment (start 106.12 106.1) (end 103.58 106.1) (width 0.5) (layer "F.Cu") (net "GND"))
 (segment (start 105.6 106.62) (end 105.6 109.625) (width 0.5) (layer "F.Cu") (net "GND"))
 (segment (start 106.12 106.1) (end 105.6 106.62) (width 0.5) (layer "F.Cu") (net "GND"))
 (segment (start 108.746 108.094) (end 108.746 109.573) (width 0.5) (layer "B.Cu") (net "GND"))
 (segment (start 108.66 106.1) (end 109.7 107.14) (width 0.5) (layer "B.Cu") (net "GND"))
 (segment (start 109.7 107.14) (end 108.746 108.094) (width 0.5) (layer "B.Cu") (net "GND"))
 (segment (start 118.82 106.1) (end 116.28 106.1) (width 0.5) (layer "B.Cu") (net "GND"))
 (segment (start 108.66 106.1) (end 106.12 106.1) (width 0.5) (layer "B.Cu") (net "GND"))
 (segment (start 104.6057 107.5759) (end 104.0333 108.1483) (width 0.2) (layer "B.Cu") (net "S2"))
 (segment (start 104.6057 102.5343) (end 104.6057 107.5759) (width 0.2) (layer "B.Cu") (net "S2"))
 (segment (start 106.12 101.02) (end 104.6057 102.5343) (width 0.2) (layer "B.Cu") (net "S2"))
 (segment (start 104.0333 109.625) (end 104.0333 108.1483) (width 0.2) (layer "B.Cu") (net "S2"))
 (segment (start 113.74 101.02) (end 115.1853 102.4653) (width 0.2) (layer "F.Cu") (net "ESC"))
 (segment (start 115.1853 103.9543) (end 116.2362 105.0052) (width 0.2) (layer "F.Cu") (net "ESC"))
 (segment (start 116.2362 105.0052) (end 116.6743 105.0052) (width 0.2) (layer "F.Cu") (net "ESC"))
 (segment (start 116.6743 105.0052) (end 117.7253 106.0562) (width 0.2) (layer "F.Cu") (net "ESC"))
 (segment (start 117.7253 106.0562) (end 117.7253 106.8183) (width 0.2) (layer "F.Cu") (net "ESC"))
 (segment (start 115.1853 102.4653) (end 115.1853 103.9543) (width 0.2) (layer "F.Cu") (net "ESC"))
 (via (at 117.7253 106.8183) (size 0.6) (drill 0.3) (layers "F.Cu" "B.Cu") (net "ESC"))
 (segment (start 117 109.625) (end 117 108.1483) (width 0.2) (layer "B.Cu") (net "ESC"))
 (segment (start 117 108.1483) (end 117.7253 107.423) (width 0.2) (layer "B.Cu") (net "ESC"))
 (segment (start 117.7253 107.423) (end 117.7253 106.8183) (width 0.2) (layer "B.Cu") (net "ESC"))
 (segment (start 108.66 101.02) (end 107.3094 102.3706) (width 0.2) (layer "B.Cu") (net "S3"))
 (segment (start 106.1501 105.0052) (end 105.7535 105.0052) (width 0.2) (layer "B.Cu") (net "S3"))
 (segment (start 107.3094 102.3706) (end 107.3094 103.8459) (width 0.2) (layer "B.Cu") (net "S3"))
 (segment (start 105.0902 105.6685) (end 105.0902 106.5086) (width 0.2) (layer "B.Cu") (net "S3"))
 (segment (start 106.7667 109.625) (end 106.7667 108.1483) (width 0.2) (layer "B.Cu") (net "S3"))
 (segment (start 106.7299 108.1483) (end 106.7667 108.1483) (width 0.2) (layer "B.Cu") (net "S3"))
 (segment (start 105.7535 105.0052) (end 105.0902 105.6685) (width 0.2) (layer "B.Cu") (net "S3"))
 (segment (start 105.0902 106.5086) (end 106.7299 108.1483) (width 0.2) (layer "B.Cu") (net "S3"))
 (segment (start 107.3094 103.8459) (end 106.1501 105.0052) (width 0.2) (layer "B.Cu") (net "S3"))
 (segment (start 118.858 105.0552) (end 119.236 105.0552) (width 0.2) (layer "B.Cu") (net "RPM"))
 (segment (start 119.8414 107.3569) (end 119.05 108.1483) (width 0.2) (layer "B.Cu") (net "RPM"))
 (segment (start 119.8414 105.6606) (end 119.8414 107.3569) (width 0.2) (layer "B.Cu") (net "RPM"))
 (segment (start 119.05 109.625) (end 119.05 108.1483) (width 0.2) (layer "B.Cu") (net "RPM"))
 (segment (start 119.236 105.0552) (end 119.8414 105.6606) (width 0.2) (layer "B.Cu") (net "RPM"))
 (segment (start 117.55 102.29) (end 117.55 103.7472) (width 0.2) (layer "B.Cu") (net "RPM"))
 (segment (start 116.28 101.02) (end 117.55 102.29) (width 0.2) (layer "B.Cu") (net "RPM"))
 (segment (start 117.55 103.7472) (end 118.858 105.0552) (width 0.2) (layer "B.Cu") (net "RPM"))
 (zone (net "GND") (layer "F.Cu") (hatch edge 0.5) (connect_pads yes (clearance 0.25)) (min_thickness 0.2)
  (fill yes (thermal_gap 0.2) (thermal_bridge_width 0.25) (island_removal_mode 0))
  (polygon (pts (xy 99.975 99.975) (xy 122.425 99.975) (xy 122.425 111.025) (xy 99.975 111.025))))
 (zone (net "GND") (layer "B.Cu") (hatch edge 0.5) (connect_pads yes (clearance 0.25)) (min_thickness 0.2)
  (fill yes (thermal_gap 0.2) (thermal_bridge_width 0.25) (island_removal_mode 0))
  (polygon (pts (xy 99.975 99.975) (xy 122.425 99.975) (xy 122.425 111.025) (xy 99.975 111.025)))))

